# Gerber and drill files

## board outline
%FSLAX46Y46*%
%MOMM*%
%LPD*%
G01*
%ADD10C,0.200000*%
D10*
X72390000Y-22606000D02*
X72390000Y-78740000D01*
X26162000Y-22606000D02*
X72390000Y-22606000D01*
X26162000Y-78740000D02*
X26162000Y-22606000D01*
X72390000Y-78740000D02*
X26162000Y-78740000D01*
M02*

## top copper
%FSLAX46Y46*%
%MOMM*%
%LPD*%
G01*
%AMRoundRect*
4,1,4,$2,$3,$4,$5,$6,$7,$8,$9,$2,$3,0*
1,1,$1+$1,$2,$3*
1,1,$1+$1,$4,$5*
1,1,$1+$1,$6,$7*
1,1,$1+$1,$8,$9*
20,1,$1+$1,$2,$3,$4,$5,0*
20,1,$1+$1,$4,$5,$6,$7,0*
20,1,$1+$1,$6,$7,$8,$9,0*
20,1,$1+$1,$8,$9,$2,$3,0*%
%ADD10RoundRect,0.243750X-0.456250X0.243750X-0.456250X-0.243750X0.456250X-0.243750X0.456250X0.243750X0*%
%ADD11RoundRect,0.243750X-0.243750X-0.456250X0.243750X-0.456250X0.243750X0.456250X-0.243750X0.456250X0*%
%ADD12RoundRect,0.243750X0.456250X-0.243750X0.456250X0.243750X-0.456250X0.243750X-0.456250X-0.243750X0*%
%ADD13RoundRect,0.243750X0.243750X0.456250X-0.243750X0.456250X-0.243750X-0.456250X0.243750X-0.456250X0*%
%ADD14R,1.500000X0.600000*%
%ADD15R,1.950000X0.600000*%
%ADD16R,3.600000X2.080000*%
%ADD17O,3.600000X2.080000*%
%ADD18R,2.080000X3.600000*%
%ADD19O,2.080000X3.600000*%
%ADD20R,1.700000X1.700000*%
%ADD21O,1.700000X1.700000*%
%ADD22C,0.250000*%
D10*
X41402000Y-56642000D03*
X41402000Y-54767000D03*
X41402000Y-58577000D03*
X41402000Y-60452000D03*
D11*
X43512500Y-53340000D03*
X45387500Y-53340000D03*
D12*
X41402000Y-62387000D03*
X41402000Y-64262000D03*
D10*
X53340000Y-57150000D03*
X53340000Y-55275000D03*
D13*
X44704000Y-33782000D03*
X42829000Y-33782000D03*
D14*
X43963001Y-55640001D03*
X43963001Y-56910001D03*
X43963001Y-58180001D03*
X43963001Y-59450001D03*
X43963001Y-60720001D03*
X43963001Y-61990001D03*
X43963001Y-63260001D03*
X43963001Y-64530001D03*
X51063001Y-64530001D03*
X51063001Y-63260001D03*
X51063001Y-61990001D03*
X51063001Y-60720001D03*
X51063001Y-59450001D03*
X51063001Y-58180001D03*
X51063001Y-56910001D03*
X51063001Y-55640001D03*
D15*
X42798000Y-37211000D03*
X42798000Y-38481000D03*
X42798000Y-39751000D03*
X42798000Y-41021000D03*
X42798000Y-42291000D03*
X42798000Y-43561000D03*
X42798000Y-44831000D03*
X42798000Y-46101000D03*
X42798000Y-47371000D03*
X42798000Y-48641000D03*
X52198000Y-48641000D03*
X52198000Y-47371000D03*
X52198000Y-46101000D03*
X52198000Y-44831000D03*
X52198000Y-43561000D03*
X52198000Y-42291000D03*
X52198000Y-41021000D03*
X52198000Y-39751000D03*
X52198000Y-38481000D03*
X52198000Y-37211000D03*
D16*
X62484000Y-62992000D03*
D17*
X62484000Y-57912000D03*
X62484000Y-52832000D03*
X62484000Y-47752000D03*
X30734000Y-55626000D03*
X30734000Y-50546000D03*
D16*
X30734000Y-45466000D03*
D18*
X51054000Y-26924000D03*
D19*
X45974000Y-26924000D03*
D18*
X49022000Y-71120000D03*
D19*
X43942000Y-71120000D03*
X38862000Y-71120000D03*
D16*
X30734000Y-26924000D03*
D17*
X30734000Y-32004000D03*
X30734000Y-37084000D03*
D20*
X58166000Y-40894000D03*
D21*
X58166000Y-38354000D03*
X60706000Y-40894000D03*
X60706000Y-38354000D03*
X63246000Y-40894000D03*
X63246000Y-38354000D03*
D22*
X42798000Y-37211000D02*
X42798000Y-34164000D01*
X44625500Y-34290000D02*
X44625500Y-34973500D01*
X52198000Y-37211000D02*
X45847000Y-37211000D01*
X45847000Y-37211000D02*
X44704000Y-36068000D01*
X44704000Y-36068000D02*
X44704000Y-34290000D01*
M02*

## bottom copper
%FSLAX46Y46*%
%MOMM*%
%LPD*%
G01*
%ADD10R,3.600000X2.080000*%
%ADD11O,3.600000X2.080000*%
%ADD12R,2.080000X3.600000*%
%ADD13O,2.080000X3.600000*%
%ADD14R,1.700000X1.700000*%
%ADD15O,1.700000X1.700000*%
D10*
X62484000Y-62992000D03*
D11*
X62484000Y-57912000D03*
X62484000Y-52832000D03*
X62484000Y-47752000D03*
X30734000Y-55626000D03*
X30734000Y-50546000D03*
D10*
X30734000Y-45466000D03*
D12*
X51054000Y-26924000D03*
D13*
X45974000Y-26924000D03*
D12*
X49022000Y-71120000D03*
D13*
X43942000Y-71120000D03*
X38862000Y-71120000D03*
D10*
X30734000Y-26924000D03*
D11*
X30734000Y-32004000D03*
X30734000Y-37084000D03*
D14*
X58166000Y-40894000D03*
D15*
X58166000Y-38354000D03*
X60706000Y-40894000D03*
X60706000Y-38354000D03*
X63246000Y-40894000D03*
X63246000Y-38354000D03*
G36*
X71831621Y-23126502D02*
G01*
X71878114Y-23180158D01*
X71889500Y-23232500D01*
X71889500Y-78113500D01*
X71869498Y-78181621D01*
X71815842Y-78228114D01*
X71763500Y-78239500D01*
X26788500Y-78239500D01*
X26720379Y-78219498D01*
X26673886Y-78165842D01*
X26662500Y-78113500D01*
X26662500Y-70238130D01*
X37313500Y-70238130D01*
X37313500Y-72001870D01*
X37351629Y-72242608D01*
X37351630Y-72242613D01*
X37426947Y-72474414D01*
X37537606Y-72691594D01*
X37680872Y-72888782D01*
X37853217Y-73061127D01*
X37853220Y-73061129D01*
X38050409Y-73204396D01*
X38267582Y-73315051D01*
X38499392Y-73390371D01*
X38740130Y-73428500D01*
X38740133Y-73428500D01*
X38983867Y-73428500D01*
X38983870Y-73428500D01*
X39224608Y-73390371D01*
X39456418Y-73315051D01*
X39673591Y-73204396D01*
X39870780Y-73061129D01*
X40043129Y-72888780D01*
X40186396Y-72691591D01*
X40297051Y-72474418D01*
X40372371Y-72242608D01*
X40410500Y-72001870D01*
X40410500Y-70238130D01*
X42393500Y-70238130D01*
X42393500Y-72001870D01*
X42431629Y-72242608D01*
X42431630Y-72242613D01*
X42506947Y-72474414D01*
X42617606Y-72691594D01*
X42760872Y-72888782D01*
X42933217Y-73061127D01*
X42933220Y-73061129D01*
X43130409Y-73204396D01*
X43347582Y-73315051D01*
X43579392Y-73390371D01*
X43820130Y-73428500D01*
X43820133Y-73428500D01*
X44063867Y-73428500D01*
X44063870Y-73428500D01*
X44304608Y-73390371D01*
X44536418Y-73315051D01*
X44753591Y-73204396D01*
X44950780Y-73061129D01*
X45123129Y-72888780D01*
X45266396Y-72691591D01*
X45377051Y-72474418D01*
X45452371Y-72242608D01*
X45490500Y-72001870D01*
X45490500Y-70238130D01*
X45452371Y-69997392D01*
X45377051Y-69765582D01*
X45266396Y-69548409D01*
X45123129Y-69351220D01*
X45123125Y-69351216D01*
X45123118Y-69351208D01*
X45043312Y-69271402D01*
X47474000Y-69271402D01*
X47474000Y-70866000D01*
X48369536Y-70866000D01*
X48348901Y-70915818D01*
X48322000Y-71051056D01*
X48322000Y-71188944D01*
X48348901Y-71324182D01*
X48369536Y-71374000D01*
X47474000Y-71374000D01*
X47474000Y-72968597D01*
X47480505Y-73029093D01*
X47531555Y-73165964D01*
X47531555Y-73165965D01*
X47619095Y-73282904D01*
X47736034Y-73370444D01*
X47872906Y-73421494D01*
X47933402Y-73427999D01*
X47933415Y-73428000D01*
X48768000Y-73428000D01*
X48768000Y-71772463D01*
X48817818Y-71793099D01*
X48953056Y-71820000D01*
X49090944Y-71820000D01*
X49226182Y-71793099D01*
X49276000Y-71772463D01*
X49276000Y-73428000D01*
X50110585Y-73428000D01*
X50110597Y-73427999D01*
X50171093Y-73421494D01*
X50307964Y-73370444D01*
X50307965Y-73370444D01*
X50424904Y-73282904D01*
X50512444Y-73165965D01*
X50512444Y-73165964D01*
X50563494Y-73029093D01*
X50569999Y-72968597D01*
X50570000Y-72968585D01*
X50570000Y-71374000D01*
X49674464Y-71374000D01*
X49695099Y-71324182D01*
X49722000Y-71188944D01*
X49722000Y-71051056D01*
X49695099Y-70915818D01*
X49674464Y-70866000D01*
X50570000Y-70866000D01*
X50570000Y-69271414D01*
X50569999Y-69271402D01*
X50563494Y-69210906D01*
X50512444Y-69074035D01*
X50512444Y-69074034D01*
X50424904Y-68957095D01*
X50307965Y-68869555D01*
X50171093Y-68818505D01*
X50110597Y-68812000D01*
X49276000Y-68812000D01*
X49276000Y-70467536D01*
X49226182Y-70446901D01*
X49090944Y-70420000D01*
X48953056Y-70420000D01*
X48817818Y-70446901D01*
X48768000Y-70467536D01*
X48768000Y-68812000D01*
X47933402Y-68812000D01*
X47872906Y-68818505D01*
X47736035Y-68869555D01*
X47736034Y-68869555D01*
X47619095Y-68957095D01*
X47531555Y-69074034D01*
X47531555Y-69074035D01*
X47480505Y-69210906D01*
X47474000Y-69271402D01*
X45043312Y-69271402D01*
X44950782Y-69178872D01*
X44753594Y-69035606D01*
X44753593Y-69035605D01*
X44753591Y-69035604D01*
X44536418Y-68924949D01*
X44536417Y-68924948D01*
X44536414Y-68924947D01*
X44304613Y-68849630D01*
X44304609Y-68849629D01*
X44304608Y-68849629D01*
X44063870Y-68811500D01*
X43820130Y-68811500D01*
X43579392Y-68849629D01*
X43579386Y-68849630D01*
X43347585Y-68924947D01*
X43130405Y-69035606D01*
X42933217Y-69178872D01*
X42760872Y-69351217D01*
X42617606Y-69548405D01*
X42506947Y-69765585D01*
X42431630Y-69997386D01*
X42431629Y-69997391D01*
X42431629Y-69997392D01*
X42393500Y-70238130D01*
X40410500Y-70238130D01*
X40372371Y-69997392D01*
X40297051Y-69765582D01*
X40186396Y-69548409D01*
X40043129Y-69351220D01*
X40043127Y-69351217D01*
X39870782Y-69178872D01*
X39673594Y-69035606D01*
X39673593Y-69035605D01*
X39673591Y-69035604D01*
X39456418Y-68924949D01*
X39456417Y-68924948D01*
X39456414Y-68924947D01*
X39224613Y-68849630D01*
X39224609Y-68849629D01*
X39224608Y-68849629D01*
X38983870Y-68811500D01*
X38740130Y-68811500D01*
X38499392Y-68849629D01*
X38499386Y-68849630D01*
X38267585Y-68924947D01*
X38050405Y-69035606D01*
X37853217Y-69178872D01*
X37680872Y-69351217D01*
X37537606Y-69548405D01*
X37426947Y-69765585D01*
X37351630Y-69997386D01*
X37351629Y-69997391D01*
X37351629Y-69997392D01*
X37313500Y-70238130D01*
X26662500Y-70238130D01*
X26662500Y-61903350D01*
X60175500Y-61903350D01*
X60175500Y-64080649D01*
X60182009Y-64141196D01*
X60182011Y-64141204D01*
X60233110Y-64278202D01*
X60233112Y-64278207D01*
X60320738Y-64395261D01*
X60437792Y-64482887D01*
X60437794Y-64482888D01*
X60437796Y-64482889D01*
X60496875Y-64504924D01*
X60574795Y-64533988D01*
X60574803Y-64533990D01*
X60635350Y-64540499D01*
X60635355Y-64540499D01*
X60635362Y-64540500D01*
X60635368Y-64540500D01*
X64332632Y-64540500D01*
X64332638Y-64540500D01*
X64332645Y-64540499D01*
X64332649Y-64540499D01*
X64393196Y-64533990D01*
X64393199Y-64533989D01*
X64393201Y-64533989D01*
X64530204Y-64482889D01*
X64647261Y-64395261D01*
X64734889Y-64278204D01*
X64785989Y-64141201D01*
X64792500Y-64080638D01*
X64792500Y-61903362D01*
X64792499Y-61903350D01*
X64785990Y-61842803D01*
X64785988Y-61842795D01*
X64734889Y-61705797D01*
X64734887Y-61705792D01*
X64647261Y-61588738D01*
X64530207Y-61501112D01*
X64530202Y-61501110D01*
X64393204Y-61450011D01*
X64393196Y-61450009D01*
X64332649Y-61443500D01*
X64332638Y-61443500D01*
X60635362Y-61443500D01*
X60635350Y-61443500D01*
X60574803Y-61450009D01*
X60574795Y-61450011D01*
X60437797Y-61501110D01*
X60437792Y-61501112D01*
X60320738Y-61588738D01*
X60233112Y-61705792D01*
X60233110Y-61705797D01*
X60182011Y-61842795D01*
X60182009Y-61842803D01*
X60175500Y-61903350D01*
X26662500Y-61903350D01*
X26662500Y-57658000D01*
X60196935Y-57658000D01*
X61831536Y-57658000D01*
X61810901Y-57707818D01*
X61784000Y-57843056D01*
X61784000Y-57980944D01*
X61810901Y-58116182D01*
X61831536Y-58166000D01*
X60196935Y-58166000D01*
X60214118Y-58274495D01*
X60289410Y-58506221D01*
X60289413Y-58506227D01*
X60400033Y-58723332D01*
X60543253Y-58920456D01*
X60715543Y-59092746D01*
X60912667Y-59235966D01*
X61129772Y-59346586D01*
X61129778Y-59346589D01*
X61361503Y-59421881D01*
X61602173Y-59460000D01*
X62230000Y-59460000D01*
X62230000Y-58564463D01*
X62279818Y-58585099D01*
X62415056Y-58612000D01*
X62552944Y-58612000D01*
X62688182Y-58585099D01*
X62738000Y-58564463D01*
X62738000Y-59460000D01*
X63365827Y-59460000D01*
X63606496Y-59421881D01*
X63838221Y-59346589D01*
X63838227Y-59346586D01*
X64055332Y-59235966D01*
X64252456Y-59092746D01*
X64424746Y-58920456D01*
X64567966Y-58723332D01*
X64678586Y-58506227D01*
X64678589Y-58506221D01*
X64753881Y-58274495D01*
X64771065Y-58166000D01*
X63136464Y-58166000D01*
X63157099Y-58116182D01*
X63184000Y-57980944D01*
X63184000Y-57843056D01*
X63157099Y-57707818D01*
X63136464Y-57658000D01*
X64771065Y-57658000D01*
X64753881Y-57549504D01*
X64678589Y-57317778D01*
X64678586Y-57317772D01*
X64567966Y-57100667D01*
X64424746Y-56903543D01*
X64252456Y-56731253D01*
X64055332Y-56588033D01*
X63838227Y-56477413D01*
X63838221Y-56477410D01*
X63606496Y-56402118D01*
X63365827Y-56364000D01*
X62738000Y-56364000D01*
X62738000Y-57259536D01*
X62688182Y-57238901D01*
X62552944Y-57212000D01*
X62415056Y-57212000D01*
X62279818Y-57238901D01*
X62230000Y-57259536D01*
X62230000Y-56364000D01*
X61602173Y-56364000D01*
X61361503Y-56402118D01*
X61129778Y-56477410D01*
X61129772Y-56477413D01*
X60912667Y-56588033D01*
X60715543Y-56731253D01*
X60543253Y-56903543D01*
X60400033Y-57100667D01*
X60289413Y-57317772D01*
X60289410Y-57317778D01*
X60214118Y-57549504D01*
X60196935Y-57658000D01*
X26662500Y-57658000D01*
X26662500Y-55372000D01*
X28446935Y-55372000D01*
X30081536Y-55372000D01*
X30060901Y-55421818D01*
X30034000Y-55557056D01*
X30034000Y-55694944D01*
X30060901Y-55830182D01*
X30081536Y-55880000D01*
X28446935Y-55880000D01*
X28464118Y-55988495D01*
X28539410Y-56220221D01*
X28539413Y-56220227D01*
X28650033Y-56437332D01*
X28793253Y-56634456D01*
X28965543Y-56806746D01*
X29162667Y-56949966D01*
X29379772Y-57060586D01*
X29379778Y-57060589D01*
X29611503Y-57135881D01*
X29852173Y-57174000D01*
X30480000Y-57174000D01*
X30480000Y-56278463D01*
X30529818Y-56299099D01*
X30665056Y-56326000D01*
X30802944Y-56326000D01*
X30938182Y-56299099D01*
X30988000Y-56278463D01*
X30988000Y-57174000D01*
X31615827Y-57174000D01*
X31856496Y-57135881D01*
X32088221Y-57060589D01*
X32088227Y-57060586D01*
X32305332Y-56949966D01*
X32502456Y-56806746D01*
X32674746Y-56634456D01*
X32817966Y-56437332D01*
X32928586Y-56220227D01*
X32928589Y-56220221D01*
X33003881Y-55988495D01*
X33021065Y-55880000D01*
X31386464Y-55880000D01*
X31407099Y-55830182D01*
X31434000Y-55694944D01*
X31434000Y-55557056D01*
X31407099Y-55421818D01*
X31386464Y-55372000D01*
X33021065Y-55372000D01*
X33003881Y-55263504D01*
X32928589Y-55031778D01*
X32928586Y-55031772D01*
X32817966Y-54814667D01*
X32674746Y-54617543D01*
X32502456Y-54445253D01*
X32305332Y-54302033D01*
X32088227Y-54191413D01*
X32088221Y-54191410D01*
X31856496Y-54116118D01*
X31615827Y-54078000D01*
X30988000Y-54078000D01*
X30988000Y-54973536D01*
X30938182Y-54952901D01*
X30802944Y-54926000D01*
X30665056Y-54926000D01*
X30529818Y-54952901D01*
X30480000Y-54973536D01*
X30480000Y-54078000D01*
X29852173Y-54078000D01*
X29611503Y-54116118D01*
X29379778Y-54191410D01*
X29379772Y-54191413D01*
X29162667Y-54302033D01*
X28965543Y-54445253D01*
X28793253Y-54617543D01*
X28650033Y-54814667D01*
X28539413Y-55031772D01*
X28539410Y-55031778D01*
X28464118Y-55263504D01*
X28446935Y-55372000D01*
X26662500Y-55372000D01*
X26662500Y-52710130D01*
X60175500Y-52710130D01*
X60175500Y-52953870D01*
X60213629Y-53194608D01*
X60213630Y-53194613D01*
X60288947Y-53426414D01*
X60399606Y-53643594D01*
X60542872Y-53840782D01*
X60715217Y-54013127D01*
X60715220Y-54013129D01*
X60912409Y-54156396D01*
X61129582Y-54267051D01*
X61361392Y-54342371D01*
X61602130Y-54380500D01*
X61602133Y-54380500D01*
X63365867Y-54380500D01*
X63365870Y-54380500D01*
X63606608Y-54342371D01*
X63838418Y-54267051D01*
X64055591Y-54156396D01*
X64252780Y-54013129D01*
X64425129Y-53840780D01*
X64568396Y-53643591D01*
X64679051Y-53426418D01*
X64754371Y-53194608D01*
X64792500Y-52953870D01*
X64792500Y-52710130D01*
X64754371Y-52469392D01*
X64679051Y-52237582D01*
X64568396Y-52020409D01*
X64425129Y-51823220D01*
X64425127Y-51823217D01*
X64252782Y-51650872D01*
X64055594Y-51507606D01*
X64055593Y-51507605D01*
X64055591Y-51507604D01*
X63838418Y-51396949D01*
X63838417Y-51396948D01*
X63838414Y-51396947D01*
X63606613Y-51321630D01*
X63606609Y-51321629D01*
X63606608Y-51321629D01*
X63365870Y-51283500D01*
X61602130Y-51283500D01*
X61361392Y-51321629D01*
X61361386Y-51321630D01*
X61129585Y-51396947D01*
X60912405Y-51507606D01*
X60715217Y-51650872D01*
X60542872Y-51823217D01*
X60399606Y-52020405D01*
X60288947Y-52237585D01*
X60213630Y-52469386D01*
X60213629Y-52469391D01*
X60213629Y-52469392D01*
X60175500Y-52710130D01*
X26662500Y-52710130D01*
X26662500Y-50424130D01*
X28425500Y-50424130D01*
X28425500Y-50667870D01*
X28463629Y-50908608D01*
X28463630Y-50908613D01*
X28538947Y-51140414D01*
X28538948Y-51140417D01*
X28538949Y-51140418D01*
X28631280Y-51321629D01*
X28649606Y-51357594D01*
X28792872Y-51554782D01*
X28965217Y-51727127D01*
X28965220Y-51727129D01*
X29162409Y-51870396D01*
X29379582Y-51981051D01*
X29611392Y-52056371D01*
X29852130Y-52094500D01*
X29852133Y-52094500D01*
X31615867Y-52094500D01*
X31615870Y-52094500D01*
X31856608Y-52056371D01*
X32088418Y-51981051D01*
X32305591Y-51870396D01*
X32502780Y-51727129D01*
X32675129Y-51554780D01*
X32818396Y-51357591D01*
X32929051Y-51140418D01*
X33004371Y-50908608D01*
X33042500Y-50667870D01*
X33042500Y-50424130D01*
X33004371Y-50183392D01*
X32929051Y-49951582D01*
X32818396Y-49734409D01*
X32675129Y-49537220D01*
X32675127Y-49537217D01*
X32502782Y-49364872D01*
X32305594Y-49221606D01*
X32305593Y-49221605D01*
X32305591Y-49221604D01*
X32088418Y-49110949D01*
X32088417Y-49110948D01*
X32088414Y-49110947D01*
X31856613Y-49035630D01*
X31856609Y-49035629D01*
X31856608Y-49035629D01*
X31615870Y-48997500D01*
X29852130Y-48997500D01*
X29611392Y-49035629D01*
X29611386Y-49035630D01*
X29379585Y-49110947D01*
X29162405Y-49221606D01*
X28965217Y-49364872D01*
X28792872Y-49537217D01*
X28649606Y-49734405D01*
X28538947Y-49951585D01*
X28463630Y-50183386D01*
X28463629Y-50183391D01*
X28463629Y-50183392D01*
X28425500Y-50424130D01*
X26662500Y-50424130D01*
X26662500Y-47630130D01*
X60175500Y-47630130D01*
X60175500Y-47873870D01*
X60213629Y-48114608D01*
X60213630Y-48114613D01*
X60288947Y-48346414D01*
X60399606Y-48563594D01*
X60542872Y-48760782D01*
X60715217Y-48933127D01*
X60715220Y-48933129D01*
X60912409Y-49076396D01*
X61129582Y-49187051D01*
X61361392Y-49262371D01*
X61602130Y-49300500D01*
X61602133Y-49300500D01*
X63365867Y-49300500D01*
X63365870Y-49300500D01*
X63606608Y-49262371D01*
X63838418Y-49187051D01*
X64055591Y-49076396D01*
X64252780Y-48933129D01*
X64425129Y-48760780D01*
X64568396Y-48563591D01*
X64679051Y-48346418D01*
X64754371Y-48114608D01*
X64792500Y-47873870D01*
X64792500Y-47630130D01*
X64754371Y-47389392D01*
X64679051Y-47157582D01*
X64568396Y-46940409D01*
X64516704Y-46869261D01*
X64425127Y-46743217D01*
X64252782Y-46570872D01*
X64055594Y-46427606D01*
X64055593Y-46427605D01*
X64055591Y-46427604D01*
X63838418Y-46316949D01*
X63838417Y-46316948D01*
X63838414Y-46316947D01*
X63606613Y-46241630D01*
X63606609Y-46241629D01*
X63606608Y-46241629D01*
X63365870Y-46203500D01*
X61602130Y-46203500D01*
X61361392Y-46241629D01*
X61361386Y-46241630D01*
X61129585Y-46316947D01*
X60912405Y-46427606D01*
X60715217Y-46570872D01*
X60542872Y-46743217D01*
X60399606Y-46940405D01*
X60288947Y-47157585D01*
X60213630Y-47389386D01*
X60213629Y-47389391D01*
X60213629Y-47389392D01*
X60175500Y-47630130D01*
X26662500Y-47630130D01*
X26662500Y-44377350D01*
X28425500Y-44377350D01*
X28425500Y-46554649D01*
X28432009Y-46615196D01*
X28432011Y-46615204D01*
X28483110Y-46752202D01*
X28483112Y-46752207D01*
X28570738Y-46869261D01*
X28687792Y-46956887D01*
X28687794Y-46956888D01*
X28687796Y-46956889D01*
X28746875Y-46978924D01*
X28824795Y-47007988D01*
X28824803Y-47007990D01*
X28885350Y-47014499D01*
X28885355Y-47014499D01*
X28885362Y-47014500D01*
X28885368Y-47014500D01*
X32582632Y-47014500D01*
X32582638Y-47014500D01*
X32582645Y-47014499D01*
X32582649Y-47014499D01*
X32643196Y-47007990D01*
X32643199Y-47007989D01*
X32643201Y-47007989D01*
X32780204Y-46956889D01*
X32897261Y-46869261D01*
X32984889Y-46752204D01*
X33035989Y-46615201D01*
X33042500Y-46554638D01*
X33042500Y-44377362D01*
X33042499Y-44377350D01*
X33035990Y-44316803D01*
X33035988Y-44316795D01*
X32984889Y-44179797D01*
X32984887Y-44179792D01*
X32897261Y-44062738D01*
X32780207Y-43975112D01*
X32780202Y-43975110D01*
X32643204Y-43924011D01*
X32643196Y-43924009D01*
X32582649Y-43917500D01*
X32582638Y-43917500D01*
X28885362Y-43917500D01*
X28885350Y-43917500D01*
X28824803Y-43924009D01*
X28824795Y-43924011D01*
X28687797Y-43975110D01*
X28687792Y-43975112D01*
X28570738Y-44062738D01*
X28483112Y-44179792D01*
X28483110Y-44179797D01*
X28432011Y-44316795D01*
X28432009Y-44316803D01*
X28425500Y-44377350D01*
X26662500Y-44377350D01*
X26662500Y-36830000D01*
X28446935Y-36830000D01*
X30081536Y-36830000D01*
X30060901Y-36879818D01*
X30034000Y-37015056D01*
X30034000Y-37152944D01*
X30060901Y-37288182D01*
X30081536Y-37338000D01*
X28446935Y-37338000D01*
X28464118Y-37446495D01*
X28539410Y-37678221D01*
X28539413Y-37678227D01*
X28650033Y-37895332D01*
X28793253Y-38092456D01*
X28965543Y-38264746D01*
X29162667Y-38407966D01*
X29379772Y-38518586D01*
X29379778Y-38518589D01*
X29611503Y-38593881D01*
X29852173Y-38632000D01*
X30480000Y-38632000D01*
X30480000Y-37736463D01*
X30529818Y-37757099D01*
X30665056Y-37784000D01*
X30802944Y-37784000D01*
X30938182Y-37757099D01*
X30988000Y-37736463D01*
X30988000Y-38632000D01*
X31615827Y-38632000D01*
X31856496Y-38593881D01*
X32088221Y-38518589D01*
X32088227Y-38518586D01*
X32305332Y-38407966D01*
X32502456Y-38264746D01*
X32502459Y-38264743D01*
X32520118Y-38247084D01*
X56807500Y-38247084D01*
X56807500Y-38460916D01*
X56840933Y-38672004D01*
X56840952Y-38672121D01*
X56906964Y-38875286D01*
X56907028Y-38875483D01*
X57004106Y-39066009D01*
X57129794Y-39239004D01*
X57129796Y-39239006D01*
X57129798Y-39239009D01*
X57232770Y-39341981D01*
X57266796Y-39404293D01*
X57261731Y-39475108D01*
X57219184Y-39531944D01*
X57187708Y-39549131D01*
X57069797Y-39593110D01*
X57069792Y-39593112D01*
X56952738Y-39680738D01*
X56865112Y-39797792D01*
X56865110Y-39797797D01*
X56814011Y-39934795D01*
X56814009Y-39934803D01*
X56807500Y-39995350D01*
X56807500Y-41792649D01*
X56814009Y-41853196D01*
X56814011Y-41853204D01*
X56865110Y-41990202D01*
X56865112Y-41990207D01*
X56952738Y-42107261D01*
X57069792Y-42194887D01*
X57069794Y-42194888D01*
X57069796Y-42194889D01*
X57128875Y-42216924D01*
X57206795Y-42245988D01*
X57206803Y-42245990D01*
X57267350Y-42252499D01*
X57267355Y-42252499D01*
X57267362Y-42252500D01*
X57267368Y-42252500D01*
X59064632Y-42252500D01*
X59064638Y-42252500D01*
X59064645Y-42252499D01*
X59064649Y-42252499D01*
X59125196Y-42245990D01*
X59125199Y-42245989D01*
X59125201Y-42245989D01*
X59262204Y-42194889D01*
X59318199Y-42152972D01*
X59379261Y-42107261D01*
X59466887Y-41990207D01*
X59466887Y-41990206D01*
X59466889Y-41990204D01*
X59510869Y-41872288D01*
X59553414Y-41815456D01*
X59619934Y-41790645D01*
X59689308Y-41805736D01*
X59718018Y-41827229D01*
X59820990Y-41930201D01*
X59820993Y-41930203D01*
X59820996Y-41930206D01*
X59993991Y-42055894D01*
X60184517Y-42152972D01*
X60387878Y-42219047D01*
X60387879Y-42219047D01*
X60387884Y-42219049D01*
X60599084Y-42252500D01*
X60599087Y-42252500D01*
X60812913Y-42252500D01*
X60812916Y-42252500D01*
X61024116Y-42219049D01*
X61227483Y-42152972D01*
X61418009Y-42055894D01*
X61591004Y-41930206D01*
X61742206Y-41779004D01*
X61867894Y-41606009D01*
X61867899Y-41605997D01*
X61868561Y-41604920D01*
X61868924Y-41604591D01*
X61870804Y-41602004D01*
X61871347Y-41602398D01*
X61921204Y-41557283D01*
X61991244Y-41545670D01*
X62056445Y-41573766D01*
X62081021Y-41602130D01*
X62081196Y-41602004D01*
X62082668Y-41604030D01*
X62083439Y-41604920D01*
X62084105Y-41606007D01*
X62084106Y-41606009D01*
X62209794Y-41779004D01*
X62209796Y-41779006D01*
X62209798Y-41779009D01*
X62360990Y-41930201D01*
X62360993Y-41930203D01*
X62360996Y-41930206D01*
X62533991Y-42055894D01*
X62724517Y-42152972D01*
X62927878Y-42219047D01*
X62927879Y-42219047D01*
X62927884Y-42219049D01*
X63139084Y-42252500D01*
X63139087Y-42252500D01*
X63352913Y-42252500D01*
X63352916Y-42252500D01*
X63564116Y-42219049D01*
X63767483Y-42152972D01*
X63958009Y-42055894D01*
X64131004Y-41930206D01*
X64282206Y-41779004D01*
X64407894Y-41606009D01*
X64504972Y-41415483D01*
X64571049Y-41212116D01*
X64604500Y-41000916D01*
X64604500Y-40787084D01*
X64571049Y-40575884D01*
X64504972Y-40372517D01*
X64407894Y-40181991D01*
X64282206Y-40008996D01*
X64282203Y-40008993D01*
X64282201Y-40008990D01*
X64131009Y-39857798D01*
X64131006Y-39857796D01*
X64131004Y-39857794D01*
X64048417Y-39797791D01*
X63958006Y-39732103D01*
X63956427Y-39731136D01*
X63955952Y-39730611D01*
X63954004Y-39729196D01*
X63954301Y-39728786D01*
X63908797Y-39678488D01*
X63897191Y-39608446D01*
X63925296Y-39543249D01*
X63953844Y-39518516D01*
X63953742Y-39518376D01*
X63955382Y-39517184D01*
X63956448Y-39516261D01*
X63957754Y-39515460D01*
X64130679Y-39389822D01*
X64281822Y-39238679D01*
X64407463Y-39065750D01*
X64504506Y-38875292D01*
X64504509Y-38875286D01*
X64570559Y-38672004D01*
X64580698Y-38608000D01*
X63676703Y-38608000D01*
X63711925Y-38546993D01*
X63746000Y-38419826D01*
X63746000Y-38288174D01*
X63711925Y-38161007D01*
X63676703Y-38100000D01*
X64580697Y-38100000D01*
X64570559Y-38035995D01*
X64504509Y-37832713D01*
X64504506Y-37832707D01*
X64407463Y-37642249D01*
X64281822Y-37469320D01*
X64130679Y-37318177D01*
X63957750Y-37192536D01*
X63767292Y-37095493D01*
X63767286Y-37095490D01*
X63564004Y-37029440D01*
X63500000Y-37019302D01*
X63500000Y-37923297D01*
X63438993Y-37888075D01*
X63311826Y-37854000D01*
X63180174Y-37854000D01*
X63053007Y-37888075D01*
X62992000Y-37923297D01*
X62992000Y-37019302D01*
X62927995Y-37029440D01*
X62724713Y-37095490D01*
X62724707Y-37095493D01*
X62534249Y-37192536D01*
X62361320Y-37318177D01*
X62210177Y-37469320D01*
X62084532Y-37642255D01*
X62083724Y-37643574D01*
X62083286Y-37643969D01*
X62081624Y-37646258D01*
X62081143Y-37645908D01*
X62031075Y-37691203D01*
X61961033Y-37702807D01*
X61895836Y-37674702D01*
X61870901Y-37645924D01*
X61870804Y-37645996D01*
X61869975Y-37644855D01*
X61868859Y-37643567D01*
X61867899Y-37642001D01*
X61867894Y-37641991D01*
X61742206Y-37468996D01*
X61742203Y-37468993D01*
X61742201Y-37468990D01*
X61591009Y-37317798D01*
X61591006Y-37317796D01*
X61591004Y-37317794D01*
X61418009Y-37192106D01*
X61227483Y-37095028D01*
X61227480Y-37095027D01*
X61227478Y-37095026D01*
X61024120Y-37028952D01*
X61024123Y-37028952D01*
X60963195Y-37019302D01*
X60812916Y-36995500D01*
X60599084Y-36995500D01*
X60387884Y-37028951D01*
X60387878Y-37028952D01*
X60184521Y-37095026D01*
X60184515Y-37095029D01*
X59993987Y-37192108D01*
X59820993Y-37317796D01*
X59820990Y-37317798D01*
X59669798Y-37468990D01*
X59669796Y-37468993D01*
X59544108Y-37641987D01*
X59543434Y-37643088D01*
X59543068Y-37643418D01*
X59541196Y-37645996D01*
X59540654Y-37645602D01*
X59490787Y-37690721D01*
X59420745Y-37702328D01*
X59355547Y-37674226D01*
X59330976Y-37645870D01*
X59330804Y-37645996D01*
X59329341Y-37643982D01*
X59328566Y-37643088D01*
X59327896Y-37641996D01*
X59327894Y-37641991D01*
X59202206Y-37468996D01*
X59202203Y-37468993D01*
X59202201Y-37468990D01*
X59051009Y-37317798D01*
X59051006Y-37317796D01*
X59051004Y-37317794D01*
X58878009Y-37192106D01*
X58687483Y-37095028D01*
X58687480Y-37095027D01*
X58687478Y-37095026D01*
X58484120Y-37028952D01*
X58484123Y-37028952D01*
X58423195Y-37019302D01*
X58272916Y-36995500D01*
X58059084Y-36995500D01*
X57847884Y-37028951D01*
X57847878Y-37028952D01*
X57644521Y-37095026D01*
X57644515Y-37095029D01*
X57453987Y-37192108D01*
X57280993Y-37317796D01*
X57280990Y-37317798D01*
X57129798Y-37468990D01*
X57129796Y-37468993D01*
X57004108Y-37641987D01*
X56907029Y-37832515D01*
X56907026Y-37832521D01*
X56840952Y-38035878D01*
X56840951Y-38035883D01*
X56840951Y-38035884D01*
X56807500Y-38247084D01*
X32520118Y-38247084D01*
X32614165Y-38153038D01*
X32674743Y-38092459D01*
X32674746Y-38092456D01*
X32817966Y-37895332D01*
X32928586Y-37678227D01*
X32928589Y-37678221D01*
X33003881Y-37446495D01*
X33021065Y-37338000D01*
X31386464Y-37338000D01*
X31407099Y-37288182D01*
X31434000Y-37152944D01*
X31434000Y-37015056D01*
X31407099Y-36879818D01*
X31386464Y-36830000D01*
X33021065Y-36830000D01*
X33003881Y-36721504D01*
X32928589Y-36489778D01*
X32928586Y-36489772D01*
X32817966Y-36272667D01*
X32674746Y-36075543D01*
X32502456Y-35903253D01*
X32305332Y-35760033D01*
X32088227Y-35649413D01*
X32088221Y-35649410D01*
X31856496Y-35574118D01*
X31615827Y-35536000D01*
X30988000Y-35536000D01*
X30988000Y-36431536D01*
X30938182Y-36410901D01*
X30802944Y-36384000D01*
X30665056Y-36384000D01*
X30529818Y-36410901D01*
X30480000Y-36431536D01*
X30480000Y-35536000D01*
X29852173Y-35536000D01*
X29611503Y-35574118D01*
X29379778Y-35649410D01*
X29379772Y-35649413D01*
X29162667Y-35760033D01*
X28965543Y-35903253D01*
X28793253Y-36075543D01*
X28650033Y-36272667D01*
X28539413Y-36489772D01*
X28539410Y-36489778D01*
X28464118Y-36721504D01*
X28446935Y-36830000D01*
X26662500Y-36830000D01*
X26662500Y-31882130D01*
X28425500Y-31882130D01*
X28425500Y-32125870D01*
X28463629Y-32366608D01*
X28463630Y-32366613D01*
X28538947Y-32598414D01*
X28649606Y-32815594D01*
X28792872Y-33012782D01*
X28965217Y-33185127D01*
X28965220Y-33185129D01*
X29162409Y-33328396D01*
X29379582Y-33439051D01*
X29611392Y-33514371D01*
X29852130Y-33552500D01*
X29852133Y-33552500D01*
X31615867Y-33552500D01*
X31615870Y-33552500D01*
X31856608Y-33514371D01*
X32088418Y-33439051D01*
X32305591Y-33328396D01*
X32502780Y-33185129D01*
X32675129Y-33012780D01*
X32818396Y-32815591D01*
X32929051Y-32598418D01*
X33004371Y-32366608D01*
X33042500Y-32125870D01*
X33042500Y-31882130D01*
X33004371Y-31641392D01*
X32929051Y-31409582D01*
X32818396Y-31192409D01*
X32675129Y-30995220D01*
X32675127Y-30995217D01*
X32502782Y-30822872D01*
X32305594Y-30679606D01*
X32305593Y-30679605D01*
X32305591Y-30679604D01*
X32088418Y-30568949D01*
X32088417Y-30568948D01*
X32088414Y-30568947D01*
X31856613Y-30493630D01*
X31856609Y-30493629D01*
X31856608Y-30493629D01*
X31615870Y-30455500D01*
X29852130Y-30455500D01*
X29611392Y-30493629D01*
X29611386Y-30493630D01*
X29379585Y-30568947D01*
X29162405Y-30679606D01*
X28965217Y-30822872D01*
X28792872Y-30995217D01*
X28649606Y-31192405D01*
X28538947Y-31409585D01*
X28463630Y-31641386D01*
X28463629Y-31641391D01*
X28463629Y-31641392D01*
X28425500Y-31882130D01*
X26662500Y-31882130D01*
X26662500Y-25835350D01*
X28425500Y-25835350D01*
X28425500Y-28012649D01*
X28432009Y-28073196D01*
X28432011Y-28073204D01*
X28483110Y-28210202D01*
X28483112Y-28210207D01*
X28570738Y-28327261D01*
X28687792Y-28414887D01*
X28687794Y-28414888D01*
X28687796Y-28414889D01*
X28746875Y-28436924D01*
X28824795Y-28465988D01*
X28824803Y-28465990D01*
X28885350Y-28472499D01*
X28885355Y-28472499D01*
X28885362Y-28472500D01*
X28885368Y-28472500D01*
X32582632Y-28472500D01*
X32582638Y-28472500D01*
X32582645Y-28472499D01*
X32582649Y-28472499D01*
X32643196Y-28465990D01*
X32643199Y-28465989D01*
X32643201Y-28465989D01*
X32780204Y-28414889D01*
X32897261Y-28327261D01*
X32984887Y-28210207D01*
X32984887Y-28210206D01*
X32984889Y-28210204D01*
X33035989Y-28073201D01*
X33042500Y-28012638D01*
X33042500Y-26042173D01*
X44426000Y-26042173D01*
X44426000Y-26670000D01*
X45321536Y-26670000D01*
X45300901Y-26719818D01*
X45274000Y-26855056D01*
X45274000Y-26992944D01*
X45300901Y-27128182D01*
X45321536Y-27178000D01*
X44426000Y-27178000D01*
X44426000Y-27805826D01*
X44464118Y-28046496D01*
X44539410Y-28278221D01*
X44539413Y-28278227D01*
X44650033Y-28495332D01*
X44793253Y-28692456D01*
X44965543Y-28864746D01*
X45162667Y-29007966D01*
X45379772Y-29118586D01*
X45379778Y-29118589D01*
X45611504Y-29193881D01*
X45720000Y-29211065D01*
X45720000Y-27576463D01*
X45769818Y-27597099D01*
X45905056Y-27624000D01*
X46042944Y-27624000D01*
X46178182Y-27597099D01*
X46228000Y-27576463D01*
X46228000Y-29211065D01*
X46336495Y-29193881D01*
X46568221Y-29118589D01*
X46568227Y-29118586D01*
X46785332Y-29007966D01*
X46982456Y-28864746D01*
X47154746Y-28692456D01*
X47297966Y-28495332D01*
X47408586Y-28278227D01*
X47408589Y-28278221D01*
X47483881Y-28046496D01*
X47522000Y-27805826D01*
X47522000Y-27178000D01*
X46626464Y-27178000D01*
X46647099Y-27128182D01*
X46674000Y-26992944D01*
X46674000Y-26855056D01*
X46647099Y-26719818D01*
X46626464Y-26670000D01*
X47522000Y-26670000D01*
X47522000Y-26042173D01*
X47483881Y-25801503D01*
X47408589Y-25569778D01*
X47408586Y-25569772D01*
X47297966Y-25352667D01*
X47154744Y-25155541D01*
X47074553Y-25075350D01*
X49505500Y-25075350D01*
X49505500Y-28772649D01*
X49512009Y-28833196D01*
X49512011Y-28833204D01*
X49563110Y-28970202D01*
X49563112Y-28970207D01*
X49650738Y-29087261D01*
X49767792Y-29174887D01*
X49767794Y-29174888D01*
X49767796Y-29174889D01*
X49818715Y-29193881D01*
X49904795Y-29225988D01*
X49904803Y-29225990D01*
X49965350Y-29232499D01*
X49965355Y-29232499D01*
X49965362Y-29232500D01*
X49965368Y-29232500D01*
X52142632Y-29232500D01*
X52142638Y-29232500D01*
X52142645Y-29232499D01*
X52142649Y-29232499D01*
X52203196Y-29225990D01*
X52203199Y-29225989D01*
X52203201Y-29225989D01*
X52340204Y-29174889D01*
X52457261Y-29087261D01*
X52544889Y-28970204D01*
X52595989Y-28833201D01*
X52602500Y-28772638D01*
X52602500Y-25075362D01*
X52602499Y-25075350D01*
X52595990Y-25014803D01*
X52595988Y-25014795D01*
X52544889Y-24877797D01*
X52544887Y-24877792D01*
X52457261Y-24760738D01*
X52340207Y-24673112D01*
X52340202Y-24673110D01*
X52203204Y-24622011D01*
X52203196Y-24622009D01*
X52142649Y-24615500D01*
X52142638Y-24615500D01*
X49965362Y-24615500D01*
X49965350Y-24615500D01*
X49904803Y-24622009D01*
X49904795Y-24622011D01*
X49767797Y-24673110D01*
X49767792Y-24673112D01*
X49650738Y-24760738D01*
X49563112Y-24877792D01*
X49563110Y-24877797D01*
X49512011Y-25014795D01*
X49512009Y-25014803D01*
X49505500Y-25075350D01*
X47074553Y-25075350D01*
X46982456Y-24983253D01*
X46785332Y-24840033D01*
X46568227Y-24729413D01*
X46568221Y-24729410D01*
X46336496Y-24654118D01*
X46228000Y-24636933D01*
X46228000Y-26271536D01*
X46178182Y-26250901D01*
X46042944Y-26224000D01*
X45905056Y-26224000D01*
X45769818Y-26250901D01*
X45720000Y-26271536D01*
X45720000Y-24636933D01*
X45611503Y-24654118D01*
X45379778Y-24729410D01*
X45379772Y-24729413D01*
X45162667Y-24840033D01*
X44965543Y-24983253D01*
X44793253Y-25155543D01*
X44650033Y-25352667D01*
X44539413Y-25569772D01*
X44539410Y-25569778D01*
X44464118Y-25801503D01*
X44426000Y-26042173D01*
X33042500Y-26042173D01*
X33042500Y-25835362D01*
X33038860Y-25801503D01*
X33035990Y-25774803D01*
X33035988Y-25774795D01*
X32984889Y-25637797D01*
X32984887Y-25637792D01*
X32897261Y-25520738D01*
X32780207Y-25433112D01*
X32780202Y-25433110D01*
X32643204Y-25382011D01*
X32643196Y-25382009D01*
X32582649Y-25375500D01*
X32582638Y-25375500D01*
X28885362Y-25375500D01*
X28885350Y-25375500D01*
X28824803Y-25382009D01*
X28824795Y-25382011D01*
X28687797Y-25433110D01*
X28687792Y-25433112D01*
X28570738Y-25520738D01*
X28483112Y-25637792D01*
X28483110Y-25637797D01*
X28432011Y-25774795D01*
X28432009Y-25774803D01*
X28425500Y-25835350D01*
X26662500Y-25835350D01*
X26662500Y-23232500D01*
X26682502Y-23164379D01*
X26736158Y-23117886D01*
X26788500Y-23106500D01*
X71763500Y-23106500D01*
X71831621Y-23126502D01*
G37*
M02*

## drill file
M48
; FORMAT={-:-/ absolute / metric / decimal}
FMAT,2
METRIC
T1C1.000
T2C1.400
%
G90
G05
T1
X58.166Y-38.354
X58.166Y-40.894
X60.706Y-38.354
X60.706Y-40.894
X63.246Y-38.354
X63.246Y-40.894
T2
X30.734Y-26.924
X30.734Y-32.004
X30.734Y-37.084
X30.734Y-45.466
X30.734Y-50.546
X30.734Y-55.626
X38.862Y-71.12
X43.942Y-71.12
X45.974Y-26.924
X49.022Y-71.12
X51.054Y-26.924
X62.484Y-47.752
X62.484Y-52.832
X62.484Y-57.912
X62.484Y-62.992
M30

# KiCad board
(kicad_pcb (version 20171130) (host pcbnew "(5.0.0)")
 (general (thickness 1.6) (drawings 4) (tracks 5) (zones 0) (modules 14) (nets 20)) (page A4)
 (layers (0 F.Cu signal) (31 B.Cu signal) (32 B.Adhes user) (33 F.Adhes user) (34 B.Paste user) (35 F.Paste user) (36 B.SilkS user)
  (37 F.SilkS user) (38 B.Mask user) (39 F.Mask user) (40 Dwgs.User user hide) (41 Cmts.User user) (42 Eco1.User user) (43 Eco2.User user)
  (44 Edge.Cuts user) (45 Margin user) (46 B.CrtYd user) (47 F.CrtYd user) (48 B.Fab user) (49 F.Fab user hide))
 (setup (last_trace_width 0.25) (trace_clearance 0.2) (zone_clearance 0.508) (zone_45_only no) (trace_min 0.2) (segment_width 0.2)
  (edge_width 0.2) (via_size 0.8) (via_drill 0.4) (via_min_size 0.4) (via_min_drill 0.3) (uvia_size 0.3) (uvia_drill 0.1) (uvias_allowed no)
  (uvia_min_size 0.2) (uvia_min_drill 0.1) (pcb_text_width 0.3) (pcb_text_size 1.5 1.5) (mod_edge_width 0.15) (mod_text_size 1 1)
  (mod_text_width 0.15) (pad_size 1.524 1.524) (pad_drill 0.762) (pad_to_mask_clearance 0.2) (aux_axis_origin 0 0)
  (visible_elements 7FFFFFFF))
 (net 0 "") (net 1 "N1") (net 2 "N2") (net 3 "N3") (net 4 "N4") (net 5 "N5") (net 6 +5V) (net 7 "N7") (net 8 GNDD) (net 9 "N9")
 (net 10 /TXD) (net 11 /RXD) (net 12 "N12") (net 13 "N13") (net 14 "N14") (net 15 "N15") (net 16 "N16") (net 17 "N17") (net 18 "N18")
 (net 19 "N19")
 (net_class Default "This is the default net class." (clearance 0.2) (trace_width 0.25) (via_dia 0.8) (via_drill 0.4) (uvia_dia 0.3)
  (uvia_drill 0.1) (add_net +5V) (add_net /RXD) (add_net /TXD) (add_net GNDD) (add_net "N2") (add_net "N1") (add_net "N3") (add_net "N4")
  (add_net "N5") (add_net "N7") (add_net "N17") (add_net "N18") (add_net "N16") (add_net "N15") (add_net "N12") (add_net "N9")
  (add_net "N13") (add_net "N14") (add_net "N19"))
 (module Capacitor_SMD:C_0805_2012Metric (layer F.Cu) (at 41.402 55.7045 270)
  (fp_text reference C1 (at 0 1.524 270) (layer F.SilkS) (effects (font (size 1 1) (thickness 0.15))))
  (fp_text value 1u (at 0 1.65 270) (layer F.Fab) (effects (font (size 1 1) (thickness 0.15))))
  (pad 2 smd roundrect (at 0.9375 0 270) (size 0.975 1.4) (layers F.Cu F.Paste F.Mask) (roundrect_rratio 0.25) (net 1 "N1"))
  (pad 1 smd roundrect (at -0.9375 0 270) (size 0.975 1.4) (layers F.Cu F.Paste F.Mask) (roundrect_rratio 0.25) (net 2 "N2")))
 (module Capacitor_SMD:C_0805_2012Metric (layer F.Cu) (at 41.402 59.5145 270)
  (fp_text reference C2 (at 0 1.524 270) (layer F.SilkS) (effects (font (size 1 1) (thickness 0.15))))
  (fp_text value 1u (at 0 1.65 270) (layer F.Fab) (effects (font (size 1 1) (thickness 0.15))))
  (pad 1 smd roundrect (at -0.9375 0 270) (size 0.975 1.4) (layers F.Cu F.Paste F.Mask) (roundrect_rratio 0.25) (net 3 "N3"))
  (pad 2 smd roundrect (at 0.9375 0 270) (size 0.975 1.4) (layers F.Cu F.Paste F.Mask) (roundrect_rratio 0.25) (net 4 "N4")))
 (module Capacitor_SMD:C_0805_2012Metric (layer F.Cu) (at 44.45 53.34)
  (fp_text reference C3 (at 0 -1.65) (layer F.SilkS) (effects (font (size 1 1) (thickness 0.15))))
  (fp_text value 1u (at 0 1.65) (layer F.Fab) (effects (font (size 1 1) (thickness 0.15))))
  (pad 1 smd roundrect (at -0.9375 0) (size 0.975 1.4) (layers F.Cu F.Paste F.Mask) (roundrect_rratio 0.25) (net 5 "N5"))
  (pad 2 smd roundrect (at 0.9375 0) (size 0.975 1.4) (layers F.Cu F.Paste F.Mask) (roundrect_rratio 0.25) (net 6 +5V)))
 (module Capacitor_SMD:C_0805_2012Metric (layer F.Cu) (at 41.402 63.3245 90)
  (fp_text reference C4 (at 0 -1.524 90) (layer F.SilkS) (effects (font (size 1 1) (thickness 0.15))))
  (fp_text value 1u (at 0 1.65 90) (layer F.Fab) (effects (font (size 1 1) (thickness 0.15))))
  (pad 2 smd roundrect (at 0.9375 0 90) (size 0.975 1.4) (layers F.Cu F.Paste F.Mask) (roundrect_rratio 0.25) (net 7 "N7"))
  (pad 1 smd roundrect (at -0.9375 0 90) (size 0.975 1.4) (layers F.Cu F.Paste F.Mask) (roundrect_rratio 0.25) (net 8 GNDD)))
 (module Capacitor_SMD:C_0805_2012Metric (layer F.Cu) (at 53.34 56.2125 270)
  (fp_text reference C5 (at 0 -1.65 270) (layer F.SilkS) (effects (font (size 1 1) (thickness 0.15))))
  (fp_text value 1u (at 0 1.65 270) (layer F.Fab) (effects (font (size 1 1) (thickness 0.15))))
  (pad 2 smd roundrect (at 0.9375 0 270) (size 0.975 1.4) (layers F.Cu F.Paste F.Mask) (roundrect_rratio 0.25) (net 8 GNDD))
  (pad 1 smd roundrect (at -0.9375 0 270) (size 0.975 1.4) (layers F.Cu F.Paste F.Mask) (roundrect_rratio 0.25) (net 6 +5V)))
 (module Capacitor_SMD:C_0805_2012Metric (layer F.Cu) (at 43.7665 33.782 180)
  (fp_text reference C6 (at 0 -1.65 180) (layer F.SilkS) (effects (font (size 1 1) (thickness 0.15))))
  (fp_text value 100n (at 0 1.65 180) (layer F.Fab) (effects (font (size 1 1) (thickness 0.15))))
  (pad 1 smd roundrect (at -0.9375 0 180) (size 0.975 1.4) (layers F.Cu F.Paste F.Mask) (roundrect_rratio 0.25) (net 8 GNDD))
  (pad 2 smd roundrect (at 0.9375 0 180) (size 0.975 1.4) (layers F.Cu F.Paste F.Mask) (roundrect_rratio 0.25) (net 6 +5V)))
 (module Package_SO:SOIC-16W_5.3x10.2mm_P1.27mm (layer F.Cu) (at 47.513001 60.085001)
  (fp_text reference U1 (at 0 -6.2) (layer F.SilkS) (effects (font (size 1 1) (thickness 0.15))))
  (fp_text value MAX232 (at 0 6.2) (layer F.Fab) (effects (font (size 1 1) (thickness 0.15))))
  (pad 1 smd rect (at -3.55 -4.445) (size 1.5 0.6) (layers F.Cu F.Paste F.Mask) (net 2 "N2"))
  (pad 2 smd rect (at -3.55 -3.175) (size 1.5 0.6) (layers F.Cu F.Paste F.Mask) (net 5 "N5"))
  (pad 3 smd rect (at -3.55 -1.905) (size 1.5 0.6) (layers F.Cu F.Paste F.Mask) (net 1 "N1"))
  (pad 4 smd rect (at -3.55 -0.635) (size 1.5 0.6) (layers F.Cu F.Paste F.Mask) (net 3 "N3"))
  (pad 5 smd rect (at -3.55 0.635) (size 1.5 0.6) (layers F.Cu F.Paste F.Mask) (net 4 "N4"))
  (pad 6 smd rect (at -3.55 1.905) (size 1.5 0.6) (layers F.Cu F.Paste F.Mask) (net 7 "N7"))
  (pad 7 smd rect (at -3.55 3.175) (size 1.5 0.6) (layers F.Cu F.Paste F.Mask) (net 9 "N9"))
  (pad 8 smd rect (at -3.55 4.445) (size 1.5 0.6) (layers F.Cu F.Paste F.Mask))
  (pad 9 smd rect (at 3.55 4.445) (size 1.5 0.6) (layers F.Cu F.Paste F.Mask))
  (pad 10 smd rect (at 3.55 3.175) (size 1.5 0.6) (layers F.Cu F.Paste F.Mask) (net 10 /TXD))
  (pad 11 smd rect (at 3.55 1.905) (size 1.5 0.6) (layers F.Cu F.Paste F.Mask))
  (pad 12 smd rect (at 3.55 0.635) (size 1.5 0.6) (layers F.Cu F.Paste F.Mask) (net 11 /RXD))
  (pad 13 smd rect (at 3.55 -0.635) (size 1.5 0.6) (layers F.Cu F.Paste F.Mask) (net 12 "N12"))
  (pad 14 smd rect (at 3.55 -1.905) (size 1.5 0.6) (layers F.Cu F.Paste F.Mask))
  (pad 15 smd rect (at 3.55 -3.175) (size 1.5 0.6) (layers F.Cu F.Paste F.Mask) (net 8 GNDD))
  (pad 16 smd rect (at 3.55 -4.445) (size 1.5 0.6) (layers F.Cu F.Paste F.Mask) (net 6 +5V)))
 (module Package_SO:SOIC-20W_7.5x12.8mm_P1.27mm (layer F.Cu) (at 47.498 42.926)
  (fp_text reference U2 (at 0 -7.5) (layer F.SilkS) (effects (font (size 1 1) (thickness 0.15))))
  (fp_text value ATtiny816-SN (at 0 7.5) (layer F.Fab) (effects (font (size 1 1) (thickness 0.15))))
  (pad 1 smd rect (at -4.7 -5.715) (size 1.95 0.6) (layers F.Cu F.Paste F.Mask) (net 6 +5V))
  (pad 2 smd rect (at -4.7 -4.445) (size 1.95 0.6) (layers F.Cu F.Paste F.Mask))
  (pad 3 smd rect (at -4.7 -3.175) (size 1.95 0.6) (layers F.Cu F.Paste F.Mask))
  (pad 4 smd rect (at -4.7 -1.905) (size 1.95 0.6) (layers F.Cu F.Paste F.Mask) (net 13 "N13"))
  (pad 5 smd rect (at -4.7 -0.635) (size 1.95 0.6) (layers F.Cu F.Paste F.Mask) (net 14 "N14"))
  (pad 6 smd rect (at -4.7 0.635) (size 1.95 0.6) (layers F.Cu F.Paste F.Mask))
  (pad 7 smd rect (at -4.7 1.905) (size 1.95 0.6) (layers F.Cu F.Paste F.Mask))
  (pad 8 smd rect (at -4.7 3.175) (size 1.95 0.6) (layers F.Cu F.Paste F.Mask) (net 11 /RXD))
  (pad 9 smd rect (at -4.7 4.445) (size 1.95 0.6) (layers F.Cu F.Paste F.Mask) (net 10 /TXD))
  (pad 10 smd rect (at -4.7 5.715) (size 1.95 0.6) (layers F.Cu F.Paste F.Mask) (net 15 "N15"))
  (pad 11 smd rect (at 4.7 5.715) (size 1.95 0.6) (layers F.Cu F.Paste F.Mask) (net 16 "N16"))
  (pad 12 smd rect (at 4.7 4.445) (size 1.95 0.6) (layers F.Cu F.Paste F.Mask) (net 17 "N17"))
  (pad 13 smd rect (at 4.7 3.175) (size 1.95 0.6) (layers F.Cu F.Paste F.Mask) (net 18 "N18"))
  (pad 14 smd rect (at 4.7 1.905) (size 1.95 0.6) (layers F.Cu F.Paste F.Mask))
  (pad 15 smd rect (at 4.7 0.635) (size 1.95 0.6) (layers F.Cu F.Paste F.Mask))
  (pad 16 smd rect (at 4.7 -0.635) (size 1.95 0.6) (layers F.Cu F.Paste F.Mask) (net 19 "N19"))
  (pad 17 smd rect (at 4.7 -1.905) (size 1.95 0.6) (layers F.Cu F.Paste F.Mask))
  (pad 18 smd rect (at 4.7 -3.175) (size 1.95 0.6) (layers F.Cu F.Paste F.Mask))
  (pad 19 smd rect (at 4.7 -4.445) (size 1.95 0.6) (layers F.Cu F.Paste F.Mask))
  (pad 20 smd rect (at 4.7 -5.715) (size 1.95 0.6) (layers F.Cu F.Paste F.Mask) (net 8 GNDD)))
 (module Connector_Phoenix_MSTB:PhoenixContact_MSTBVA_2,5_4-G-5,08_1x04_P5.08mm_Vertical (layer F.Cu) (at 62.484 62.992 90)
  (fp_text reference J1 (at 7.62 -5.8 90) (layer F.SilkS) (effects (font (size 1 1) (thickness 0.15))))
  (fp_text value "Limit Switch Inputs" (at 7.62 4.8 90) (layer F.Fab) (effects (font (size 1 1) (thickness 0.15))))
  (pad 1 thru_hole rect (at 0 0 90) (size 2.08 3.6) (drill 1.4) (layers *.Cu *.Mask) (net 6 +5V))
  (pad 2 thru_hole oval (at 5.08 0 90) (size 2.08 3.6) (drill 1.4) (layers *.Cu *.Mask) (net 8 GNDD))
  (pad 3 thru_hole oval (at 10.16 0 90) (size 2.08 3.6) (drill 1.4) (layers *.Cu *.Mask) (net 17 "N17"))
  (pad 4 thru_hole oval (at 15.24 0 90) (size 2.08 3.6) (drill 1.4) (layers *.Cu *.Mask) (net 18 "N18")))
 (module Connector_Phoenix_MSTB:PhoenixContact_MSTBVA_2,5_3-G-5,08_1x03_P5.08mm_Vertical (layer F.Cu) (at 30.734 45.466 270)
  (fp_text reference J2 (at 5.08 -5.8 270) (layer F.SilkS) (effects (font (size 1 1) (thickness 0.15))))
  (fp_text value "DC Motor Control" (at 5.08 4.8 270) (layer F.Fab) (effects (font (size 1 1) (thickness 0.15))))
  (pad 3 thru_hole oval (at 10.16 0 270) (size 2.08 3.6) (drill 1.4) (layers *.Cu *.Mask) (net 8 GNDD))
  (pad 2 thru_hole oval (at 5.08 0 270) (size 2.08 3.6) (drill 1.4) (layers *.Cu *.Mask) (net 15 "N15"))
  (pad 1 thru_hole rect (at 0 0 270) (size 2.08 3.6) (drill 1.4) (layers *.Cu *.Mask) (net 16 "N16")))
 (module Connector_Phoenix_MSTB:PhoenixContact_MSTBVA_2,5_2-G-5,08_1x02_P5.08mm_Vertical (layer F.Cu) (at 51.054 26.924 180)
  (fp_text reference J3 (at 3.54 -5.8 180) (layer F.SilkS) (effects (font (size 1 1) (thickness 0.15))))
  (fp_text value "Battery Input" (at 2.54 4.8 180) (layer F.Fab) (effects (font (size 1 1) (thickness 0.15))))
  (pad 1 thru_hole rect (at 0 0 180) (size 2.08 3.6) (drill 1.4) (layers *.Cu *.Mask) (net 6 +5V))
  (pad 2 thru_hole oval (at 5.08 0 180) (size 2.08 3.6) (drill 1.4) (layers *.Cu *.Mask) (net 8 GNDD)))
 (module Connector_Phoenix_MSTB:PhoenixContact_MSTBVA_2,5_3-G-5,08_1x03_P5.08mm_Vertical (layer F.Cu) (at 49.022 71.12 180)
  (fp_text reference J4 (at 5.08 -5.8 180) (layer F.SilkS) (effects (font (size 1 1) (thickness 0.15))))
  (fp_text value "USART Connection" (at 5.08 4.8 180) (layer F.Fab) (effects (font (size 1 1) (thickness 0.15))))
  (pad 1 thru_hole rect (at 0 0 180) (size 2.08 3.6) (drill 1.4) (layers *.Cu *.Mask) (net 8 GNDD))
  (pad 2 thru_hole oval (at 5.08 0 180) (size 2.08 3.6) (drill 1.4) (layers *.Cu *.Mask) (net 12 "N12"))
  (pad 3 thru_hole oval (at 10.16 0 180) (size 2.08 3.6) (drill 1.4) (layers *.Cu *.Mask) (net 9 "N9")))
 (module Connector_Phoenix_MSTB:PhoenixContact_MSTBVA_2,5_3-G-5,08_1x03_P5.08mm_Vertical (layer F.Cu) (at 30.734 26.924 270)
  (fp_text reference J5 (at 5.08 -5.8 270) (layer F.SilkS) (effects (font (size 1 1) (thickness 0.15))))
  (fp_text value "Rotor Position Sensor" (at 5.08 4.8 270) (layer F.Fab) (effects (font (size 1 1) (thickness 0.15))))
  (pad 1 thru_hole rect (at 0 0 270) (size 2.08 3.6) (drill 1.4) (layers *.Cu *.Mask) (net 13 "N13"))
  (pad 2 thru_hole oval (at 5.08 0 270) (size 2.08 3.6) (drill 1.4) (layers *.Cu *.Mask) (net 14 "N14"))
  (pad 3 thru_hole oval (at 10.16 0 270) (size 2.08 3.6) (drill 1.4) (layers *.Cu *.Mask) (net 8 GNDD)))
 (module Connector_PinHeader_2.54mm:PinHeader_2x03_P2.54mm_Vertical (layer F.Cu) (at 58.166 40.894 90)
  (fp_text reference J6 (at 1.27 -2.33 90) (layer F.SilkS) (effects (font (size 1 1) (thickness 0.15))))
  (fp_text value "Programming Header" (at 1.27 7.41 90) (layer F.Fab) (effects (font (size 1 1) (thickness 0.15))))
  (pad 1 thru_hole rect (at 0 0 90) (size 1.7 1.7) (drill 1) (layers *.Cu *.Mask) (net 19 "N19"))
  (pad 2 thru_hole oval (at 2.54 0 90) (size 1.7 1.7) (drill 1) (layers *.Cu *.Mask) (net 6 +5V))
  (pad 3 thru_hole oval (at 0 2.54 90) (size 1.7 1.7) (drill 1) (layers *.Cu *.Mask))
  (pad 4 thru_hole oval (at 2.54 2.54 90) (size 1.7 1.7) (drill 1) (layers *.Cu *.Mask))
  (pad 5 thru_hole oval (at 0 5.08 90) (size 1.7 1.7) (drill 1) (layers *.Cu *.Mask))
  (pad 6 thru_hole oval (at 2.54 5.08 90) (size 1.7 1.7) (drill 1) (layers *.Cu *.Mask) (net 8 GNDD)))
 (gr_line (start 72.39 22.606) (end 72.39 78.74) (layer Edge.Cuts) (width 0.2))
 (gr_line (start 26.162 22.606) (end 72.39 22.606) (layer Edge.Cuts) (width 0.2))
 (gr_line (start 26.162 78.74) (end 26.162 22.606) (layer Edge.Cuts) (width 0.2))
 (gr_line (start 72.39 78.74) (end 26.162 78.74) (layer Edge.Cuts) (width 0.2))
 (segment (start 42.798 37.211) (end 42.798 34.164) (width 0.25) (layer F.Cu) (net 6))
 (segment (start 44.6255 34.29) (end 44.6255 34.9735) (width 0.25) (layer F.Cu) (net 8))
 (segment (start 52.198 37.211) (end 45.847 37.211) (width 0.25) (layer F.Cu) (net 8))
 (segment (start 45.847 37.211) (end 44.704 36.068) (width 0.25) (layer F.Cu) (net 8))
 (segment (start 44.704 36.068) (end 44.704 34.29) (width 0.25) (layer F.Cu) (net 8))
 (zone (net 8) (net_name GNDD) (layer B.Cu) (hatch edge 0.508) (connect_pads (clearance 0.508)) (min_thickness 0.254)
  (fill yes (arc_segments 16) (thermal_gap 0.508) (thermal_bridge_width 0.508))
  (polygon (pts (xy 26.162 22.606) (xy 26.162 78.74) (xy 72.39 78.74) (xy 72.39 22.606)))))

